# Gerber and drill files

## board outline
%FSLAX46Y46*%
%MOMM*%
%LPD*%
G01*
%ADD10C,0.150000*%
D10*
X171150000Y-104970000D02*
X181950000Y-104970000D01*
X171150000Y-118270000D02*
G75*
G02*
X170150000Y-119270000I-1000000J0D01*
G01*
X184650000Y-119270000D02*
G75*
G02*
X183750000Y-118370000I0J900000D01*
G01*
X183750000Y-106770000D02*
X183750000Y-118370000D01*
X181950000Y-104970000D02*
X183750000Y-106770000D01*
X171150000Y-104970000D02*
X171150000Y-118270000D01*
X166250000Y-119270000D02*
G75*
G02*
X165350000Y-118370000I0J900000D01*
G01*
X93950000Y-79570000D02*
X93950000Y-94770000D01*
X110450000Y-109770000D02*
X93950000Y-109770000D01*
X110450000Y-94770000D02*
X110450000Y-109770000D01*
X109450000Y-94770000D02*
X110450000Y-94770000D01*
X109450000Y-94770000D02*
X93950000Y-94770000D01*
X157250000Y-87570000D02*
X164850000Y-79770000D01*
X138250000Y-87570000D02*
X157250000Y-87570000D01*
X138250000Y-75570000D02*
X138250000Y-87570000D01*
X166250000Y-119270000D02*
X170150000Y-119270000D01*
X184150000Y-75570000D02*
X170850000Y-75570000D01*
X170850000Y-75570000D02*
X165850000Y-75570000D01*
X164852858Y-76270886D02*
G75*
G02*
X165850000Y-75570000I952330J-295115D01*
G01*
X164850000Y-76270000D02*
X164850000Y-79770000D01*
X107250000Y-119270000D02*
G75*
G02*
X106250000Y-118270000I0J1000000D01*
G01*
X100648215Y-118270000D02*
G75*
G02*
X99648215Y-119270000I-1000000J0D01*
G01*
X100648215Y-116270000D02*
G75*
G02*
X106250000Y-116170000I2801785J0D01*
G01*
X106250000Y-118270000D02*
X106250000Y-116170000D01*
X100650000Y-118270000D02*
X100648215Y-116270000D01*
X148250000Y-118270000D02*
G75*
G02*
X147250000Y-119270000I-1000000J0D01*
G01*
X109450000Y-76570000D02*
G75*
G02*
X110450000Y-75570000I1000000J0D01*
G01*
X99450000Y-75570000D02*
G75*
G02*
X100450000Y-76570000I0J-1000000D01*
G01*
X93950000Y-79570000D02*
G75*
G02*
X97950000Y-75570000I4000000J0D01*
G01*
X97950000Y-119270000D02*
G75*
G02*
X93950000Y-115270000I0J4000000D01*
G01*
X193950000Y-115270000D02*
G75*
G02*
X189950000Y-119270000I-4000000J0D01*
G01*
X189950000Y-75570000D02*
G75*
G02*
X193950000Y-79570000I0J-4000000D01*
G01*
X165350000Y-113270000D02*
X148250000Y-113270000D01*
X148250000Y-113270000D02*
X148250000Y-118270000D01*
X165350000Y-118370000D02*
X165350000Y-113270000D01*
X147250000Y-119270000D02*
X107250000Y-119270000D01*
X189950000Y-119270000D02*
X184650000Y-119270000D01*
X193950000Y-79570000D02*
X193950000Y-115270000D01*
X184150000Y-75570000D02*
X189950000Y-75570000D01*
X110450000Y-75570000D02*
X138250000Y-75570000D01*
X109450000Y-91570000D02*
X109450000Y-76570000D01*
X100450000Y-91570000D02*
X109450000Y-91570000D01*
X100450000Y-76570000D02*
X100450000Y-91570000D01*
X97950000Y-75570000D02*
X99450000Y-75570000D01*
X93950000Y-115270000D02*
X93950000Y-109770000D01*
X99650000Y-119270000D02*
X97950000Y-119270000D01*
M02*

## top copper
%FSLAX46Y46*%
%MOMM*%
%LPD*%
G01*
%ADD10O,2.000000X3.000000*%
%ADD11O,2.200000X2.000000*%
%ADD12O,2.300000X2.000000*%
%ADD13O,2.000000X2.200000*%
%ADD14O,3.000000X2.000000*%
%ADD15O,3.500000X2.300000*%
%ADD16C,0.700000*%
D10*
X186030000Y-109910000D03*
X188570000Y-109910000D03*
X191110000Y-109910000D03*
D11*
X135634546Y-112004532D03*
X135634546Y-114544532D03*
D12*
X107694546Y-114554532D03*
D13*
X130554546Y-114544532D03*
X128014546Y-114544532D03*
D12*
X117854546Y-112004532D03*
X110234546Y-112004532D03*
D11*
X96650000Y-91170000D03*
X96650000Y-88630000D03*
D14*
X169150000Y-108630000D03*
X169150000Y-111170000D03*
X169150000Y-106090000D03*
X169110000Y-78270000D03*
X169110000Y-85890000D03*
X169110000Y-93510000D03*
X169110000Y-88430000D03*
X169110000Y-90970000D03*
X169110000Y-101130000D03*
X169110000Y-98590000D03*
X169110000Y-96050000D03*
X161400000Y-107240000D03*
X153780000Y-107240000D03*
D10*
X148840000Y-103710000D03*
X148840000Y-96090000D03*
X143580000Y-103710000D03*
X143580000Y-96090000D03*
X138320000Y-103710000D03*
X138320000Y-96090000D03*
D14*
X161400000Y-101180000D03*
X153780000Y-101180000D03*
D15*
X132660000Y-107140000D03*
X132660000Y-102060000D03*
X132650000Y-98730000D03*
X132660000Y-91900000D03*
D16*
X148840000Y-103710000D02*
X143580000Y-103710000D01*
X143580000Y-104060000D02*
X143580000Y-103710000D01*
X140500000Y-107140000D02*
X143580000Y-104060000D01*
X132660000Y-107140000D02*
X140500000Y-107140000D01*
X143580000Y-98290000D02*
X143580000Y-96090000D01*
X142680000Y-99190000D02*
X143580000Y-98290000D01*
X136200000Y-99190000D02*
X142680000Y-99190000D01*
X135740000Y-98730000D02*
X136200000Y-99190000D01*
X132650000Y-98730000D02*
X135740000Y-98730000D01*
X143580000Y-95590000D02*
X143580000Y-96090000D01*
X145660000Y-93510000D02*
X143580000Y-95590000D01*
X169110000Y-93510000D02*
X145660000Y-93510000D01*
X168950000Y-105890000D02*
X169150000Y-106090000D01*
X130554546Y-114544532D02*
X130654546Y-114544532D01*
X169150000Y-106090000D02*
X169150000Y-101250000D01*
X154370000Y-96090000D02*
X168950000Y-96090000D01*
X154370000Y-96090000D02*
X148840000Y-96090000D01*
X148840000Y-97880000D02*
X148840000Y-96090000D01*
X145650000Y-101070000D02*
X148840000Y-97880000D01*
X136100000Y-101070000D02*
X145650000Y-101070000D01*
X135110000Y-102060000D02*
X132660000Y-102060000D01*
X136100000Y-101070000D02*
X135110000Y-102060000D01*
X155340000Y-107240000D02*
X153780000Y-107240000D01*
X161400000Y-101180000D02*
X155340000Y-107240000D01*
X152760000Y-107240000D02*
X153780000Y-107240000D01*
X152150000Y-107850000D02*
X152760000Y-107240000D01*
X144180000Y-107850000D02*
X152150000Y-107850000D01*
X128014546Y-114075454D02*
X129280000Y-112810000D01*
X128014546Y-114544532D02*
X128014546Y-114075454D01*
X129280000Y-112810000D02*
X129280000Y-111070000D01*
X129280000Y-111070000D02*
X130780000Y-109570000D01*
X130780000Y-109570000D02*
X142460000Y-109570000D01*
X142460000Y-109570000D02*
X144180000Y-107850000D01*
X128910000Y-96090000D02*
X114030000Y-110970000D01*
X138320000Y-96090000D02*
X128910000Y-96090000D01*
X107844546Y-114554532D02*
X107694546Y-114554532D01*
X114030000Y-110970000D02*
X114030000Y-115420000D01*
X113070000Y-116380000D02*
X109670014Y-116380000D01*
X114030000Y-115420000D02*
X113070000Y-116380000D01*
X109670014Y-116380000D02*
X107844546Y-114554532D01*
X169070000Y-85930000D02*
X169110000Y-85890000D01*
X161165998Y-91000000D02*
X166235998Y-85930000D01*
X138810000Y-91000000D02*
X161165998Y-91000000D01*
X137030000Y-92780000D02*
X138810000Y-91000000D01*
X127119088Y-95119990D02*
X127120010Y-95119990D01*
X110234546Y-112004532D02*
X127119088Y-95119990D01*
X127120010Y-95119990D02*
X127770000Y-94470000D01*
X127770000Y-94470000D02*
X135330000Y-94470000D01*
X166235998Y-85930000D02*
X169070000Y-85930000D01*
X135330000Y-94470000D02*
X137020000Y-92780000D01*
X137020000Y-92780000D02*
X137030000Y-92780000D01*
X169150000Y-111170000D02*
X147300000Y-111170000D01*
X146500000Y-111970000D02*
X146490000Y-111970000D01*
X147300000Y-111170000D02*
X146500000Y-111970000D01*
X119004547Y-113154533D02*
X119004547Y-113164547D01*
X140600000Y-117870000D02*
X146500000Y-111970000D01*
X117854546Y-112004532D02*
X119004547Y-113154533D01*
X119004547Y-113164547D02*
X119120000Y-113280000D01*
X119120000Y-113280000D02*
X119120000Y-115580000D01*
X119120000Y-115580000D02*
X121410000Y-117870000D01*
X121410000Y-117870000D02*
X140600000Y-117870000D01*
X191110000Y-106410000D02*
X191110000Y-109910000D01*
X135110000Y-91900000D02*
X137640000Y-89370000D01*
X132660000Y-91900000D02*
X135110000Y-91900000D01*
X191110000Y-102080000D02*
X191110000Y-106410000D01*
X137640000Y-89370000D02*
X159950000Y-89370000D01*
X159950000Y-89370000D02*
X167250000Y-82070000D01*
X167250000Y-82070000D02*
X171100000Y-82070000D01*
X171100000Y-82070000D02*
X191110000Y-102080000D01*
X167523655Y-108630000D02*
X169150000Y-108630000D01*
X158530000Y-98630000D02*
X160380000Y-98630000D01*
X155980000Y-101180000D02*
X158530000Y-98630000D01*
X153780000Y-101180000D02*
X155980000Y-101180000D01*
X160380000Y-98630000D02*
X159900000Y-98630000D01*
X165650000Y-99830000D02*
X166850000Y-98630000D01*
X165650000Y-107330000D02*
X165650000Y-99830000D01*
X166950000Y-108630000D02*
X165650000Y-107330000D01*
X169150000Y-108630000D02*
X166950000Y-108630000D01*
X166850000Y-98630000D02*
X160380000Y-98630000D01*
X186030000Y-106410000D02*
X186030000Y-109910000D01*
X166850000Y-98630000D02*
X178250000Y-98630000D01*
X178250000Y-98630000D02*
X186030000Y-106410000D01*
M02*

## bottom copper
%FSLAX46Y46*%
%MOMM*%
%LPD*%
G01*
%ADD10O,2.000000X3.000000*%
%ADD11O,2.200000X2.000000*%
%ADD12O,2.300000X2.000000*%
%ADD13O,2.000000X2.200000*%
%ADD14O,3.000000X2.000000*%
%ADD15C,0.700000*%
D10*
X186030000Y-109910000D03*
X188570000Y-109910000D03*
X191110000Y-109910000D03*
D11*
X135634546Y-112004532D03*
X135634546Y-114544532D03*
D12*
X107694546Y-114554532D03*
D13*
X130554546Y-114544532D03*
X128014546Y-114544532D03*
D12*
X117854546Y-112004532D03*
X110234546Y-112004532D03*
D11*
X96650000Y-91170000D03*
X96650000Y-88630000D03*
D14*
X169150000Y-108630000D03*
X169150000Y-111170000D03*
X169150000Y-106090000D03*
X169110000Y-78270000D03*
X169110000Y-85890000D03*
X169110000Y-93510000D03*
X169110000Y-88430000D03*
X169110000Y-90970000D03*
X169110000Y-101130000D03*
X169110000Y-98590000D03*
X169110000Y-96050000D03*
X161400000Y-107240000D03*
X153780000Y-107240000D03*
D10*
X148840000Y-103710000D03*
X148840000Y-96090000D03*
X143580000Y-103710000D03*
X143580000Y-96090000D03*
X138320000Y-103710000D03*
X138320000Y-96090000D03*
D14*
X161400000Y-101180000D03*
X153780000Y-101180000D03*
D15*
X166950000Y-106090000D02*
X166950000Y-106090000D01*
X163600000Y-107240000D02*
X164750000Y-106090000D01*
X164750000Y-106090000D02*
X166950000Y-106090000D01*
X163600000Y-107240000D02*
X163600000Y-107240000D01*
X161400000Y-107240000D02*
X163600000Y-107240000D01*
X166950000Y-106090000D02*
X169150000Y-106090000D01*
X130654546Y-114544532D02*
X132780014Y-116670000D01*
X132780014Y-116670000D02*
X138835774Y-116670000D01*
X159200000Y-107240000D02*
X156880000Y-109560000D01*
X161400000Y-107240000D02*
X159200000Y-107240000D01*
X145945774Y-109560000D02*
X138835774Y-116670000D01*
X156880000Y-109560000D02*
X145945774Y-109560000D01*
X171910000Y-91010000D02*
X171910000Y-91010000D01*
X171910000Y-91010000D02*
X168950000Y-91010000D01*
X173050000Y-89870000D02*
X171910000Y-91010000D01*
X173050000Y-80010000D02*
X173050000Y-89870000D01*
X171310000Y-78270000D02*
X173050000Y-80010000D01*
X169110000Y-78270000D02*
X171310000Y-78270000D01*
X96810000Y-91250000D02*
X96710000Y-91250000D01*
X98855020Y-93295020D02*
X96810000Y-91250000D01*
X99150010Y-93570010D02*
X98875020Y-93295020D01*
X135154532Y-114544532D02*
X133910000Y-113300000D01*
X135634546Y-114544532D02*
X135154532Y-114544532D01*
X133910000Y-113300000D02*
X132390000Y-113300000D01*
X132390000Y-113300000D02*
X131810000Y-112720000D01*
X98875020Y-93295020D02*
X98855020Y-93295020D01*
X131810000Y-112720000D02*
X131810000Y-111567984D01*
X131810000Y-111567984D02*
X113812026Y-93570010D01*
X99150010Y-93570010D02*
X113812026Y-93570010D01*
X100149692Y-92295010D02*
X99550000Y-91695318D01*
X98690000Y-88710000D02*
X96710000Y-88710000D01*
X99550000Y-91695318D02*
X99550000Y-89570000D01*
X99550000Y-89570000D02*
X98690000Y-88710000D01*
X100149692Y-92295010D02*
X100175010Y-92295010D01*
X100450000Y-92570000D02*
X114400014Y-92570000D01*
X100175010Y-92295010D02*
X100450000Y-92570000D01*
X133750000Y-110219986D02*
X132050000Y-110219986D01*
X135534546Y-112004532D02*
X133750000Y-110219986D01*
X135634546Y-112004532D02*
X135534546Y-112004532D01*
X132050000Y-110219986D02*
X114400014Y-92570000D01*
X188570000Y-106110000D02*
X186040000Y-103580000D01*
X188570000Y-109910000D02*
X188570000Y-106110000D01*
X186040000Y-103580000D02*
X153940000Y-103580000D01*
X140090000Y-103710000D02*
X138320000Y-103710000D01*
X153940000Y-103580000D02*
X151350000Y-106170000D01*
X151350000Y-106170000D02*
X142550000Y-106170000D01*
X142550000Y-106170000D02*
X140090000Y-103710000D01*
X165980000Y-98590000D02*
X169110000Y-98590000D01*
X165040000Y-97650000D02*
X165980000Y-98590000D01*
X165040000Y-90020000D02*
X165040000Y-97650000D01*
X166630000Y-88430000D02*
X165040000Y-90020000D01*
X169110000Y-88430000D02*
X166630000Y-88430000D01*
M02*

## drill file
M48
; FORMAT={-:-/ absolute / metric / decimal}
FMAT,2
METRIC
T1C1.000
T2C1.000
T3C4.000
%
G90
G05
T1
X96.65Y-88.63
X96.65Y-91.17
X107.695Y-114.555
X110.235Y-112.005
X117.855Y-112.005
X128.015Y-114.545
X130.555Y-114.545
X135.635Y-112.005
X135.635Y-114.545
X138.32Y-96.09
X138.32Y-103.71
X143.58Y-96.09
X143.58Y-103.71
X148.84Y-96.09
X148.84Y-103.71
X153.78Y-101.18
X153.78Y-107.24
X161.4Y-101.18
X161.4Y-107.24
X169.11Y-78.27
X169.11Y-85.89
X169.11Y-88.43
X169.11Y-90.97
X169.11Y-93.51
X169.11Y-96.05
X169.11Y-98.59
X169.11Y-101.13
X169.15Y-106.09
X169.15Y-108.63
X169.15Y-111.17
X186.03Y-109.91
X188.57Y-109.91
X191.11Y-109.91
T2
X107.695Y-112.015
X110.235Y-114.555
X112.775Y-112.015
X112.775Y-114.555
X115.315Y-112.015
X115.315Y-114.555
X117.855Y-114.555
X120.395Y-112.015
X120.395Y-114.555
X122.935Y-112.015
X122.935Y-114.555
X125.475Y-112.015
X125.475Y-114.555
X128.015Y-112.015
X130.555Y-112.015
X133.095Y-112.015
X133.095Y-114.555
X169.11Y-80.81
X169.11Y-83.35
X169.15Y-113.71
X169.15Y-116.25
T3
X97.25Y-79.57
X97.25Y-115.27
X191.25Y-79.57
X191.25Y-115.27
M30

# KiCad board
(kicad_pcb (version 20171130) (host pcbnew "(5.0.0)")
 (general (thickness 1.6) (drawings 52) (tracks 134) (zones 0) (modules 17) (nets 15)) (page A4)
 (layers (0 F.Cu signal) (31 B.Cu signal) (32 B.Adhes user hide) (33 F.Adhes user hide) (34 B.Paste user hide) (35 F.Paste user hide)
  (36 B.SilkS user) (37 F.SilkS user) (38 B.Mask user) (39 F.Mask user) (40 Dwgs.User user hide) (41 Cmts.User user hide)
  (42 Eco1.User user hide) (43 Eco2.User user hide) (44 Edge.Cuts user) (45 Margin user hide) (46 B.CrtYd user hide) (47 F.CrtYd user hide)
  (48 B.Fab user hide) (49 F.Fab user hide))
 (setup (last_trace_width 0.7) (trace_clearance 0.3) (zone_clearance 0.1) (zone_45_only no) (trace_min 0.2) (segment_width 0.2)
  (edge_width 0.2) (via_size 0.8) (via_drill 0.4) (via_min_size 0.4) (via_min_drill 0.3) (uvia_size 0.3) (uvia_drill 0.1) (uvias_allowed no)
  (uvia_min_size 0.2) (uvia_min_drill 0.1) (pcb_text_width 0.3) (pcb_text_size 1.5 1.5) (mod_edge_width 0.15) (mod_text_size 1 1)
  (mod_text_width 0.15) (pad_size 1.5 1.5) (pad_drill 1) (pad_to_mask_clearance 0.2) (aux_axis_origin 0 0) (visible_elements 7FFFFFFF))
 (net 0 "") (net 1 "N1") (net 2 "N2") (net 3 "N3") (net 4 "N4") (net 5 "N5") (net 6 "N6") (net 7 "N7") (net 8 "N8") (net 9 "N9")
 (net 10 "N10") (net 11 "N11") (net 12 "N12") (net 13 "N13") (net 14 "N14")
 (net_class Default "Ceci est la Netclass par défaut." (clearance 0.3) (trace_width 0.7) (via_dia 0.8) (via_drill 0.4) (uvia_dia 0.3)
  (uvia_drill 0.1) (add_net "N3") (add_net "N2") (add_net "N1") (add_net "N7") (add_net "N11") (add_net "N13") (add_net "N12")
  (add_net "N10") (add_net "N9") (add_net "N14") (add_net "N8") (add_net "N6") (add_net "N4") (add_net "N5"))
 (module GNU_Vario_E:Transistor (layer F.Cu) (at 193.65 107.37 180)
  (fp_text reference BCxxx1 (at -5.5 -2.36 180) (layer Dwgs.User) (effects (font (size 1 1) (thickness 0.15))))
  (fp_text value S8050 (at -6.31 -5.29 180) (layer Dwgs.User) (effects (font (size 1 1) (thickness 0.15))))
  (pad 3 thru_hole oval (at 7.62 -2.54 180) (size 2 3) (drill 1) (layers *.Cu *.Mask) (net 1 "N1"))
  (pad 2 thru_hole oval (at 5.08 -2.54 180) (size 2 3) (drill 1) (layers *.Cu *.Mask) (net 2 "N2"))
  (pad 1 thru_hole oval (at 2.54 -2.54 180) (size 2 3) (drill 1) (layers *.Cu *.Mask) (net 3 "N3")))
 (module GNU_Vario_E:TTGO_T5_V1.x (layer F.Cu) (at 136.184546 112.224532 90)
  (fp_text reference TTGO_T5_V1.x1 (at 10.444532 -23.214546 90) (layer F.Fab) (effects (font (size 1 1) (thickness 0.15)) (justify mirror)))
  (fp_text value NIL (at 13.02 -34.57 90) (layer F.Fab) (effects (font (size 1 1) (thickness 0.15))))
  (pad "" np_thru_hole circle (at 0.21 -28.49 90) (size 1 1) (drill 1) (layers *.Cu *.Mask))
  (pad "" np_thru_hole circle (at 0.21 -23.41 90) (size 1 1) (drill 1) (layers *.Cu *.Mask))
  (pad "" np_thru_hole circle (at 0.21 -20.87 90) (size 1 1) (drill 1) (layers *.Cu *.Mask))
  (pad "" np_thru_hole circle (at -2.33 -3.09 90) (size 1 1) (drill 1) (layers *.Cu *.Mask))
  (pad "" np_thru_hole circle (at 0.21 -3.09 90) (size 1 1) (drill 1) (layers *.Cu *.Mask))
  (pad "" np_thru_hole circle (at 0.21 -5.63 90) (size 1 1) (drill 1) (layers *.Cu *.Mask))
  (pad "" np_thru_hole circle (at 0.21 -15.79 90) (size 1 1) (drill 1) (layers *.Cu *.Mask))
  (pad "" np_thru_hole circle (at 0.21 -13.25 90) (size 1 1) (drill 1) (layers *.Cu *.Mask))
  (pad "" np_thru_hole circle (at 0.21 -8.17 90) (size 1 1) (drill 1) (layers *.Cu *.Mask))
  (pad "" np_thru_hole circle (at 0.21 -10.71 90) (size 1 1) (drill 1) (layers *.Cu *.Mask))
  (pad "" np_thru_hole circle (at -2.33 -10.71 90) (size 1 1) (drill 1) (layers *.Cu *.Mask))
  (pad "" np_thru_hole circle (at -2.33 -13.25 90) (size 1 1) (drill 1) (layers *.Cu *.Mask))
  (pad "" np_thru_hole circle (at -2.33 -15.79 90) (size 1 1) (drill 1) (layers *.Cu *.Mask))
  (pad "" np_thru_hole circle (at -2.33 -18.33 90) (size 1 1) (drill 1) (layers *.Cu *.Mask))
  (pad "" np_thru_hole circle (at -2.33 -20.87 90) (size 1 1) (drill 1) (layers *.Cu *.Mask))
  (pad "" np_thru_hole circle (at -2.33 -23.41 90) (size 1 1) (drill 1) (layers *.Cu *.Mask))
  (pad "" np_thru_hole circle (at -2.33 -25.95 90) (size 1 1) (drill 1) (layers *.Cu *.Mask))
  (pad 13 thru_hole oval (at 0.22 -0.55 90) (size 2 2.2) (drill 1) (layers *.Cu *.Mask) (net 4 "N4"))
  (pad 1 thru_hole oval (at -2.32 -0.55 90) (size 2 2.2) (drill 1) (layers *.Cu *.Mask) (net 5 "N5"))
  (pad 12 thru_hole oval (at -2.33 -28.49 90) (size 2 2.3) (drill 1) (layers *.Cu *.Mask) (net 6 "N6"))
  (pad 3 thru_hole oval (at -2.32 -5.63 90) (size 2.2 2) (drill 1) (layers *.Cu *.Mask) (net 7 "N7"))
  (pad 4 thru_hole oval (at -2.32 -8.17 90) (size 2.2 2) (drill 1) (layers *.Cu *.Mask) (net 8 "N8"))
  (pad 20 thru_hole oval (at 0.22 -18.33 90) (size 2 2.3) (drill 1) (layers *.Cu *.Mask) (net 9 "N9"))
  (pad 23 thru_hole oval (at 0.22 -25.95 90) (size 2 2.3) (drill 1) (layers *.Cu *.Mask) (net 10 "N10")))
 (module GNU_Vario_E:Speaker (layer F.Cu) (at 99.19 93.71 90)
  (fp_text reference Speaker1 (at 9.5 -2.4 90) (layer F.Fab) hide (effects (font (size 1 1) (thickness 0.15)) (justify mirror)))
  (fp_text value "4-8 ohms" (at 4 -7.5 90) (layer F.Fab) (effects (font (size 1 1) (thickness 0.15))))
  (pad 2 thru_hole oval (at 2.54 -2.54 90) (size 2 2.2) (drill 1) (layers *.Cu *.Mask) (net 5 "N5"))
  (pad 1 thru_hole oval (at 5.08 -2.54 90) (size 2 2.2) (drill 1) (layers *.Cu *.Mask) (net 4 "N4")))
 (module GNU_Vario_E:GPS (layer F.Cu) (at 169.15 106.09 270)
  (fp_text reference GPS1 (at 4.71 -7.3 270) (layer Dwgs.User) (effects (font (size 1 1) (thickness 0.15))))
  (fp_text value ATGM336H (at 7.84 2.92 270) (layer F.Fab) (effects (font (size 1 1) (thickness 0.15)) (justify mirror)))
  (pad 2 thru_hole oval (at 2.54 0 270) (size 2 3) (drill 1) (layers *.Cu *.Mask) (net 1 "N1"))
  (pad 3 thru_hole oval (at 5.08 0 270) (size 2 3) (drill 1) (layers *.Cu *.Mask) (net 9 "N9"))
  (pad 1 thru_hole oval (at 0 0 270) (size 2 3) (drill 1) (layers *.Cu *.Mask) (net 7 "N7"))
  (pad "" np_thru_hole circle (at 7.62 0 270) (size 1 1) (drill 1) (layers *.Cu *.Mask))
  (pad "" np_thru_hole circle (at 10.16 0 270) (size 1 1) (drill 1) (layers *.Cu *.Mask)))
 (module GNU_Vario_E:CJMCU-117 (layer F.Cu) (at 171.65 90.97 90)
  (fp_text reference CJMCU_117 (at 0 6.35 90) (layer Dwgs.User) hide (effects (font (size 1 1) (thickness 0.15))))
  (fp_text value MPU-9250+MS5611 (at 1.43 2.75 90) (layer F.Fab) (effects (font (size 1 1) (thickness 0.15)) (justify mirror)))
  (pad 10 thru_hole oval (at 12.7 -2.54 90) (size 2 3) (drill 1) (layers *.Cu *.Mask) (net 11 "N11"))
  (pad 7 thru_hole oval (at 5.08 -2.54 90) (size 2 3) (drill 1) (layers *.Cu *.Mask) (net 10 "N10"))
  (pad 4 thru_hole oval (at -2.54 -2.54 90) (size 2 3) (drill 1) (layers *.Cu *.Mask) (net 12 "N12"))
  (pad 6 thru_hole oval (at 2.54 -2.54 90) (size 2 3) (drill 1) (layers *.Cu *.Mask) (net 1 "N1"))
  (pad 5 thru_hole oval (at 0 -2.54 90) (size 2 3) (drill 1) (layers *.Cu *.Mask) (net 11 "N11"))
  (pad 1 thru_hole oval (at -10.16 -2.54 90) (size 2 3) (drill 1) (layers *.Cu *.Mask) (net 7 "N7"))
  (pad 2 thru_hole oval (at -7.62 -2.54 90) (size 2 3) (drill 1) (layers *.Cu *.Mask) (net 1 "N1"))
  (pad 3 thru_hole oval (at -5.08 -2.54 90) (size 2 3) (drill 1) (layers *.Cu *.Mask) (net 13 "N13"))
  (pad "" np_thru_hole circle (at 7.62 -2.54 90) (size 1 1) (drill 1) (layers *.Cu *.Mask))
  (pad "" np_thru_hole circle (at 10.16 -2.54 90) (size 1 1) (drill 1) (layers *.Cu *.Mask)))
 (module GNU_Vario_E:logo (layer F.Cu) (at 115.96 84.56 90)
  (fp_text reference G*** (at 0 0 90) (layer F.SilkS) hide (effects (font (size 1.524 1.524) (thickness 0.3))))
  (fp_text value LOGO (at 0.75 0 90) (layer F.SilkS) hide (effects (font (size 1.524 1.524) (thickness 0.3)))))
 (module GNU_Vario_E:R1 (layer F.Cu) (at 153.78 107.24 270)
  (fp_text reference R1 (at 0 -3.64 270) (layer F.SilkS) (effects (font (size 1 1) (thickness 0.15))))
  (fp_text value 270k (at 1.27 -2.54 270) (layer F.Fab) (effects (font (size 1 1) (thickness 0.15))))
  (pad 2 thru_hole oval (at 0 -7.62 270) (size 2 3) (drill 1) (layers *.Cu *.Mask) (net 7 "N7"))
  (pad 1 thru_hole oval (at 0 0 270) (size 2 3) (drill 1) (layers *.Cu *.Mask) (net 8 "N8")))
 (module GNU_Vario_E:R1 (layer F.Cu) (at 148.84 96.09 180)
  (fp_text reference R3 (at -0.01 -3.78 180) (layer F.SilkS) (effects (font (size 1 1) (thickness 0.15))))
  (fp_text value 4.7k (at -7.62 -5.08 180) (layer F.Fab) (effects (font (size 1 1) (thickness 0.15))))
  (pad 2 thru_hole oval (at 0 -7.62 180) (size 2 3) (drill 1) (layers *.Cu *.Mask) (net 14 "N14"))
  (pad 1 thru_hole oval (at 0 0 180) (size 2 3) (drill 1) (layers *.Cu *.Mask) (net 13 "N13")))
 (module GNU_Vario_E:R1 (layer F.Cu) (at 143.58 96.09 180)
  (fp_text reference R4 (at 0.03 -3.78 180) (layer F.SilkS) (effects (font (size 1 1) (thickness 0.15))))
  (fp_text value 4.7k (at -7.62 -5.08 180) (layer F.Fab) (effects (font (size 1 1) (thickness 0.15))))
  (pad 2 thru_hole oval (at 0 -7.62 180) (size 2 3) (drill 1) (layers *.Cu *.Mask) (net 14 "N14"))
  (pad 1 thru_hole oval (at 0 0 180) (size 2 3) (drill 1) (layers *.Cu *.Mask) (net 12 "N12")))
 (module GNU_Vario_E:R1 (layer F.Cu) (at 138.32 96.09 180)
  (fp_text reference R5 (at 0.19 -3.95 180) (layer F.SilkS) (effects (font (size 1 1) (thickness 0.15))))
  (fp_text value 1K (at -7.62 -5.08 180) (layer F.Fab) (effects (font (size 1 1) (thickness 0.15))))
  (pad 2 thru_hole oval (at 0 -7.62 180) (size 2 3) (drill 1) (layers *.Cu *.Mask) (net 2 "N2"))
  (pad 1 thru_hole oval (at 0 0 180) (size 2 3) (drill 1) (layers *.Cu *.Mask) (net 6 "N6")))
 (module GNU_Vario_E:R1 (layer F.Cu) (at 153.78 101.18 270)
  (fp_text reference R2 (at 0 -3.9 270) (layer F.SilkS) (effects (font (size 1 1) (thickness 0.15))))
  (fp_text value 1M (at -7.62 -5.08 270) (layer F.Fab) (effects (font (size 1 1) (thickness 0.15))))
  (pad 2 thru_hole oval (at 0 -7.62 270) (size 2 3) (drill 1) (layers *.Cu *.Mask) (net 8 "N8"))
  (pad 1 thru_hole oval (at 0 0 270) (size 2 3) (drill 1) (layers *.Cu *.Mask) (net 1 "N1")))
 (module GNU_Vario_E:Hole (layer F.Cu) (at 97.25 115.27)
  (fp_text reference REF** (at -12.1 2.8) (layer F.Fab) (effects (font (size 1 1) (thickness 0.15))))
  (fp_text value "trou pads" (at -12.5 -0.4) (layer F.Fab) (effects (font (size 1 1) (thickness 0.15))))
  (pad "" np_thru_hole circle (at 0 0) (size 4 4) (drill 4) (layers *.Cu *.Mask)))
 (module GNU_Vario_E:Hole (layer F.Cu) (at 97.25 79.57)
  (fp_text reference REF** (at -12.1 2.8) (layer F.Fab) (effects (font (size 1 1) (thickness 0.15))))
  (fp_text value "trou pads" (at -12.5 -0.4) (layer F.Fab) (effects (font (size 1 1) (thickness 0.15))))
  (pad "" np_thru_hole circle (at 0 0) (size 4 4) (drill 4) (layers *.Cu *.Mask)))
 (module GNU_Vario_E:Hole (layer F.Cu) (at 191.25 79.57)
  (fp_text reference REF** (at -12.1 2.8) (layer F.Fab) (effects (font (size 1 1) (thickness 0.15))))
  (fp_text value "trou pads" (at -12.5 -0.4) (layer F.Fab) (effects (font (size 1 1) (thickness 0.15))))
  (pad "" np_thru_hole circle (at 0 0) (size 4 4) (drill 4) (layers *.Cu *.Mask)))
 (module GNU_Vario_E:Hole (layer F.Cu) (at 191.25 115.27)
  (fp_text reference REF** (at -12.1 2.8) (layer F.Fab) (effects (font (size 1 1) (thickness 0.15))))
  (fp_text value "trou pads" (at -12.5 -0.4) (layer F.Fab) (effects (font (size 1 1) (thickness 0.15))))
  (pad "" np_thru_hole circle (at 0 0) (size 4 4) (drill 4) (layers *.Cu *.Mask)))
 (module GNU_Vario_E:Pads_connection (layer F.Cu) (at 132.66 94.44)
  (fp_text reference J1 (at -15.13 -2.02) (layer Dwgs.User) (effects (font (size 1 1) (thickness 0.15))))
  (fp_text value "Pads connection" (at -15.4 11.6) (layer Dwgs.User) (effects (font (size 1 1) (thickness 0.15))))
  (pad 5 smd oval (at 0 12.7) (size 3.5 2.3) (layers F.Cu F.Mask) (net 14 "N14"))
  (pad 4 smd oval (at 0 7.62) (size 3.5 2.3) (layers F.Cu F.Mask) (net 13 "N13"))
  (pad 3 smd oval (at -0.01 4.29) (size 3.5 2.3) (layers F.Cu F.Mask) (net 12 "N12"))
  (pad 1 smd oval (at 0 -2.54) (size 3.5 2.3) (layers F.Cu F.Mask) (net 3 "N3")))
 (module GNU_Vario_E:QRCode (layer B.Cu) (at 125.16 85.57)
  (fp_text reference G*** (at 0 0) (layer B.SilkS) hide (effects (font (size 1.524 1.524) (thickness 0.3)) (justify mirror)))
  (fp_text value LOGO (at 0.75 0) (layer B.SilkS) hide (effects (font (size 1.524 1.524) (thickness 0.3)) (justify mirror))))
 (gr_line (start 171.15 104.97) (end 181.95 104.97) (layer Edge.Cuts) (width 0.15))
 (gr_arc (start 170.15 118.27) (end 170.15 119.27) (angle -90) (layer Edge.Cuts) (width 0.15))
 (gr_arc (start 184.65 118.37) (end 183.75 118.37) (angle -90) (layer Edge.Cuts) (width 0.15))
 (gr_line (start 183.75 106.77) (end 183.75 118.37) (layer Edge.Cuts) (width 0.15))
 (gr_line (start 181.95 104.97) (end 183.75 106.77) (layer Edge.Cuts) (width 0.15))
 (gr_line (start 171.15 104.97) (end 171.15 118.27) (layer Edge.Cuts) (width 0.15))
 (gr_arc (start 166.25 118.37) (end 165.35 118.37) (angle -90) (layer Edge.Cuts) (width 0.15))
 (gr_line (start 93.95 79.57) (end 93.95 94.77) (layer Edge.Cuts) (width 0.15))
 (gr_line (start 110.45 109.77) (end 93.95 109.77) (layer Edge.Cuts) (width 0.15))
 (gr_line (start 110.45 94.77) (end 110.45 109.77) (layer Edge.Cuts) (width 0.15))
 (gr_line (start 109.45 94.77) (end 110.45 94.77) (layer Edge.Cuts) (width 0.15))
 (gr_line (start 109.45 94.77) (end 93.95 94.77) (layer Edge.Cuts) (width 0.15))
 (gr_line (start 157.25 87.57) (end 164.85 79.77) (layer Edge.Cuts) (width 0.15))
 (gr_line (start 138.25 87.57) (end 157.25 87.57) (layer Edge.Cuts) (width 0.15))
 (gr_line (start 138.25 75.57) (end 138.25 87.57) (layer Edge.Cuts) (width 0.15))
 (gr_line (start 166.25 119.27) (end 170.15 119.27) (layer Edge.Cuts) (width 0.15))
 (gr_line (start 184.15 75.57) (end 170.85 75.57) (layer Edge.Cuts) (width 0.15))
 (gr_line (start 170.85 75.57) (end 165.85 75.57) (layer Edge.Cuts) (width 0.15))
 (gr_arc (start 165.805188 76.566001) (end 165.85 75.57) (angle -75.35856355) (layer Edge.Cuts) (width 0.15))
 (gr_line (start 164.85 76.27) (end 164.85 79.77) (layer Edge.Cuts) (width 0.15))
 (gr_arc (start 107.25 118.27) (end 106.25 118.27) (angle -90) (layer Edge.Cuts) (width 0.15))
 (gr_arc (start 99.648215 118.27) (end 99.648215 119.27) (angle -90) (layer Edge.Cuts) (width 0.15))
 (gr_arc (start 103.45 116.27) (end 106.25 116.17) (angle -177.9545915) (layer Edge.Cuts) (width 0.15))
 (gr_line (start 106.25 118.27) (end 106.25 116.17) (layer Edge.Cuts) (width 0.15))
 (gr_line (start 100.65 118.27) (end 100.648215 116.27) (layer Edge.Cuts) (width 0.15))
 (gr_arc (start 147.25 118.27) (end 147.25 119.27) (angle -90) (layer Edge.Cuts) (width 0.15))
 (gr_arc (start 110.45 76.57) (end 110.45 75.57) (angle -90) (layer Edge.Cuts) (width 0.15))
 (gr_arc (start 99.45 76.57) (end 100.45 76.57) (angle -90) (layer Edge.Cuts) (width 0.15))
 (gr_arc (start 97.95 79.57) (end 97.95 75.57) (angle -90) (layer Edge.Cuts) (width 0.15))
 (gr_arc (start 97.95 115.27) (end 93.95 115.27) (angle -90) (layer Edge.Cuts) (width 0.15))
 (gr_arc (start 189.95 115.27) (end 189.95 119.27) (angle -90) (layer Edge.Cuts) (width 0.15))
 (gr_arc (start 189.95 79.57) (end 193.95 79.57) (angle -90) (layer Edge.Cuts) (width 0.15))
 (gr_line (start 165.35 113.27) (end 148.25 113.27) (layer Edge.Cuts) (width 0.15))
 (gr_line (start 148.25 113.27) (end 148.25 118.27) (layer Edge.Cuts) (width 0.15))
 (gr_line (start 165.35 118.37) (end 165.35 113.27) (layer Edge.Cuts) (width 0.15))
 (gr_line (start 147.25 119.27) (end 107.25 119.27) (layer Edge.Cuts) (width 0.15))
 (gr_line (start 189.95 119.27) (end 184.65 119.27) (layer Edge.Cuts) (width 0.15))
 (gr_line (start 193.95 79.57) (end 193.95 115.27) (layer Edge.Cuts) (width 0.15))
 (gr_line (start 184.15 75.57) (end 189.95 75.57) (layer Edge.Cuts) (width 0.15))
 (gr_line (start 110.45 75.57) (end 138.25 75.57) (layer Edge.Cuts) (width 0.15))
 (gr_line (start 109.45 91.57) (end 109.45 76.57) (layer Edge.Cuts) (width 0.15))
 (gr_line (start 100.45 91.57) (end 109.45 91.57) (layer Edge.Cuts) (width 0.15))
 (gr_line (start 100.45 76.57) (end 100.45 91.57) (layer Edge.Cuts) (width 0.15))
 (gr_line (start 97.95 75.57) (end 99.45 75.57) (layer Edge.Cuts) (width 0.15))
 (gr_line (start 93.95 115.27) (end 93.95 109.77) (layer Edge.Cuts) (width 0.15))
 (gr_line (start 99.65 119.27) (end 97.95 119.27) (layer Edge.Cuts) (width 0.15))
 (segment (start 148.84 103.71) (end 143.58 103.71) (width 0.7) (layer F.Cu) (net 14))
 (segment (start 143.58 104.06) (end 143.58 103.71) (width 0.7) (layer F.Cu) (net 14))
 (segment (start 140.5 107.14) (end 143.58 104.06) (width 0.7) (layer F.Cu) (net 14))
 (segment (start 132.66 107.14) (end 140.5 107.14) (width 0.7) (layer F.Cu) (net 14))
 (segment (start 143.58 98.29) (end 143.58 96.09) (width 0.7) (layer F.Cu) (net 12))
 (segment (start 142.68 99.19) (end 143.58 98.29) (width 0.7) (layer F.Cu) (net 12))
 (segment (start 136.2 99.19) (end 142.68 99.19) (width 0.7) (layer F.Cu) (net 12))
 (segment (start 135.74 98.73) (end 136.2 99.19) (width 0.7) (layer F.Cu) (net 12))
 (segment (start 132.65 98.73) (end 135.74 98.73) (width 0.7) (layer F.Cu) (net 12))
 (segment (start 143.58 95.59) (end 143.58 96.09) (width 0.7) (layer F.Cu) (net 12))
 (segment (start 145.66 93.51) (end 143.58 95.59) (width 0.7) (layer F.Cu) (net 12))
 (segment (start 169.11 93.51) (end 145.66 93.51) (width 0.7) (layer F.Cu) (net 12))
 (segment (start 168.95 105.89) (end 169.15 106.09) (width 0.7) (layer F.Cu) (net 7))
 (segment (start 166.95 106.09) (end 166.95 106.09) (width 0.7) (layer B.Cu) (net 7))
 (segment (start 163.6 107.24) (end 164.75 106.09) (width 0.7) (layer B.Cu) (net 7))
 (segment (start 164.75 106.09) (end 166.95 106.09) (width 0.7) (layer B.Cu) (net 7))
 (segment (start 163.6 107.24) (end 163.6 107.24) (width 0.7) (layer B.Cu) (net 7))
 (segment (start 161.4 107.24) (end 163.6 107.24) (width 0.7) (layer B.Cu) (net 7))
 (segment (start 166.95 106.09) (end 169.15 106.09) (width 0.7) (layer B.Cu) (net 7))
 (segment (start 130.654546 114.544532) (end 132.780014 116.67) (width 0.7) (layer B.Cu) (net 7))
 (segment (start 130.554546 114.544532) (end 130.654546 114.544532) (width 0.7) (layer F.Cu) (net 7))
 (segment (start 132.780014 116.67) (end 138.835774 116.67) (width 0.7) (layer B.Cu) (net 7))
 (segment (start 169.15 106.09) (end 169.15 101.25) (width 0.7) (layer F.Cu) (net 7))
 (segment (start 159.2 107.24) (end 156.88 109.56) (width 0.7) (layer B.Cu) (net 7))
 (segment (start 161.4 107.24) (end 159.2 107.24) (width 0.7) (layer B.Cu) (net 7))
 (segment (start 145.945774 109.56) (end 138.835774 116.67) (width 0.7) (layer B.Cu) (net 7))
 (segment (start 156.88 109.56) (end 145.945774 109.56) (width 0.7) (layer B.Cu) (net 7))
 (segment (start 154.37 96.09) (end 168.95 96.09) (width 0.7) (layer F.Cu) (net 13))
 (segment (start 154.37 96.09) (end 148.84 96.09) (width 0.7) (layer F.Cu) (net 13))
 (segment (start 148.84 97.88) (end 148.84 96.09) (width 0.7) (layer F.Cu) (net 13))
 (segment (start 145.65 101.07) (end 148.84 97.88) (width 0.7) (layer F.Cu) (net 13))
 (segment (start 136.1 101.07) (end 145.65 101.07) (width 0.7) (layer F.Cu) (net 13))
 (segment (start 135.11 102.06) (end 132.66 102.06) (width 0.7) (layer F.Cu) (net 13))
 (segment (start 136.1 101.07) (end 135.11 102.06) (width 0.7) (layer F.Cu) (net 13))
 (segment (start 155.34 107.24) (end 153.78 107.24) (width 0.7) (layer F.Cu) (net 8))
 (segment (start 161.4 101.18) (end 155.34 107.24) (width 0.7) (layer F.Cu) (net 8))
 (segment (start 152.76 107.24) (end 153.78 107.24) (width 0.7) (layer F.Cu) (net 8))
 (segment (start 152.15 107.85) (end 152.76 107.24) (width 0.7) (layer F.Cu) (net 8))
 (segment (start 144.18 107.85) (end 152.15 107.85) (width 0.7) (layer F.Cu) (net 8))
 (segment (start 128.014546 114.075454) (end 129.28 112.81) (width 0.7) (layer F.Cu) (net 8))
 (segment (start 128.014546 114.544532) (end 128.014546 114.075454) (width 0.7) (layer F.Cu) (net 8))
 (segment (start 129.28 112.81) (end 129.28 111.07) (width 0.7) (layer F.Cu) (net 8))
 (segment (start 129.28 111.07) (end 130.78 109.57) (width 0.7) (layer F.Cu) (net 8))
 (segment (start 130.78 109.57) (end 142.46 109.57) (width 0.7) (layer F.Cu) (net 8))
 (segment (start 142.46 109.57) (end 144.18 107.85) (width 0.7) (layer F.Cu) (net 8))
 (segment (start 128.91 96.09) (end 114.03 110.97) (width 0.7) (layer F.Cu) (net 6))
 (segment (start 138.32 96.09) (end 128.91 96.09) (width 0.7) (layer F.Cu) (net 6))
 (segment (start 107.844546 114.554532) (end 107.694546 114.554532) (width 0.7) (layer F.Cu) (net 6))
 (segment (start 114.03 110.97) (end 114.03 115.42) (width 0.7) (layer F.Cu) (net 6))
 (segment (start 113.07 116.38) (end 109.670014 116.38) (width 0.7) (layer F.Cu) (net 6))
 (segment (start 114.03 115.42) (end 113.07 116.38) (width 0.7) (layer F.Cu) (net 6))
 (segment (start 109.670014 116.38) (end 107.844546 114.554532) (width 0.7) (layer F.Cu) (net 6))
 (segment (start 171.91 91.01) (end 171.91 91.01) (width 0.7) (layer B.Cu) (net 11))
 (segment (start 171.91 91.01) (end 168.95 91.01) (width 0.7) (layer B.Cu) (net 11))
 (segment (start 173.05 89.87) (end 171.91 91.01) (width 0.7) (layer B.Cu) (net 11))
 (segment (start 173.05 80.01) (end 173.05 89.87) (width 0.7) (layer B.Cu) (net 11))
 (segment (start 171.31 78.27) (end 173.05 80.01) (width 0.7) (layer B.Cu) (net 11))
 (segment (start 169.11 78.27) (end 171.31 78.27) (width 0.7) (layer B.Cu) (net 11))
 (segment (start 169.07 85.93) (end 169.11 85.89) (width 0.7) (layer F.Cu) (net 10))
 (segment (start 161.165998 91) (end 166.235998 85.93) (width 0.7) (layer F.Cu) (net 10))
 (segment (start 138.81 91) (end 161.165998 91) (width 0.7) (layer F.Cu) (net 10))
 (segment (start 137.03 92.78) (end 138.81 91) (width 0.7) (layer F.Cu) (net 10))
 (segment (start 127.119088 95.11999) (end 127.12001 95.11999) (width 0.7) (layer F.Cu) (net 10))
 (segment (start 110.234546 112.004532) (end 127.119088 95.11999) (width 0.7) (layer F.Cu) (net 10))
 (segment (start 127.12001 95.11999) (end 127.77 94.47) (width 0.7) (layer F.Cu) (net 10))
 (segment (start 127.77 94.47) (end 135.33 94.47) (width 0.7) (layer F.Cu) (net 10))
 (segment (start 166.235998 85.93) (end 169.07 85.93) (width 0.7) (layer F.Cu) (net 10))
 (segment (start 135.33 94.47) (end 137.02 92.78) (width 0.7) (layer F.Cu) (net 10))
 (segment (start 137.02 92.78) (end 137.03 92.78) (width 0.7) (layer F.Cu) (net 10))
 (segment (start 169.15 111.17) (end 147.3 111.17) (width 0.7) (layer F.Cu) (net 9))
 (segment (start 146.5 111.97) (end 146.49 111.97) (width 0.7) (layer F.Cu) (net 9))
 (segment (start 147.3 111.17) (end 146.5 111.97) (width 0.7) (layer F.Cu) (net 9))
 (segment (start 119.004547 113.154533) (end 119.004547 113.164547) (width 0.7) (layer F.Cu) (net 9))
 (segment (start 140.6 117.87) (end 146.5 111.97) (width 0.7) (layer F.Cu) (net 9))
 (segment (start 117.854546 112.004532) (end 119.004547 113.154533) (width 0.7) (layer F.Cu) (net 9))
 (segment (start 119.004547 113.164547) (end 119.12 113.28) (width 0.7) (layer F.Cu) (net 9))
 (segment (start 119.12 113.28) (end 119.12 115.58) (width 0.7) (layer F.Cu) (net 9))
 (segment (start 119.12 115.58) (end 121.41 117.87) (width 0.7) (layer F.Cu) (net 9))
 (segment (start 121.41 117.87) (end 140.6 117.87) (width 0.7) (layer F.Cu) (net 9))
 (segment (start 96.81 91.25) (end 96.71 91.25) (width 0.7) (layer B.Cu) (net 5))
 (segment (start 98.85502 93.29502) (end 96.81 91.25) (width 0.7) (layer B.Cu) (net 5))
 (segment (start 99.15001 93.57001) (end 98.87502 93.29502) (width 0.7) (layer B.Cu) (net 5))
 (segment (start 135.154532 114.544532) (end 133.91 113.3) (width 0.7) (layer B.Cu) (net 5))
 (segment (start 135.634546 114.544532) (end 135.154532 114.544532) (width 0.7) (layer B.Cu) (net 5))
 (segment (start 133.91 113.3) (end 132.39 113.3) (width 0.7) (layer B.Cu) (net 5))
 (segment (start 132.39 113.3) (end 131.81 112.72) (width 0.7) (layer B.Cu) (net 5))
 (segment (start 98.87502 93.29502) (end 98.85502 93.29502) (width 0.7) (layer B.Cu) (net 5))
 (segment (start 131.81 112.72) (end 131.81 111.567984) (width 0.7) (layer B.Cu) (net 5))
 (segment (start 131.81 111.567984) (end 113.812026 93.57001) (width 0.7) (layer B.Cu) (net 5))
 (segment (start 99.15001 93.57001) (end 113.812026 93.57001) (width 0.7) (layer B.Cu) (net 5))
 (segment (start 100.149692 92.29501) (end 99.55 91.695318) (width 0.7) (layer B.Cu) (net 4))
 (segment (start 98.69 88.71) (end 96.71 88.71) (width 0.7) (layer B.Cu) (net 4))
 (segment (start 99.55 91.695318) (end 99.55 89.57) (width 0.7) (layer B.Cu) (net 4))
 (segment (start 99.55 89.57) (end 98.69 88.71) (width 0.7) (layer B.Cu) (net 4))
 (segment (start 100.149692 92.29501) (end 100.17501 92.29501) (width 0.7) (layer B.Cu) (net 4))
 (segment (start 100.45 92.57) (end 114.400014 92.57) (width 0.7) (layer B.Cu) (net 4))
 (segment (start 100.17501 92.29501) (end 100.45 92.57) (width 0.7) (layer B.Cu) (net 4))
 (segment (start 133.75 110.219986) (end 132.05 110.219986) (width 0.7) (layer B.Cu) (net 4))
 (segment (start 135.534546 112.004532) (end 133.75 110.219986) (width 0.7) (layer B.Cu) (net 4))
 (segment (start 135.634546 112.004532) (end 135.534546 112.004532) (width 0.7) (layer B.Cu) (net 4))
 (segment (start 132.05 110.219986) (end 114.400014 92.57) (width 0.7) (layer B.Cu) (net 4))
 (segment (start 191.11 106.41) (end 191.11 109.91) (width 0.7) (layer F.Cu) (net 3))
 (segment (start 135.11 91.9) (end 137.64 89.37) (width 0.7) (layer F.Cu) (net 3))
 (segment (start 132.66 91.9) (end 135.11 91.9) (width 0.7) (layer F.Cu) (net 3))
 (segment (start 191.11 102.08) (end 191.11 106.41) (width 0.7) (layer F.Cu) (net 3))
 (segment (start 137.64 89.37) (end 159.95 89.37) (width 0.7) (layer F.Cu) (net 3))
 (segment (start 159.95 89.37) (end 167.25 82.07) (width 0.7) (layer F.Cu) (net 3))
 (segment (start 167.25 82.07) (end 171.1 82.07) (width 0.7) (layer F.Cu) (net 3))
 (segment (start 171.1 82.07) (end 191.11 102.08) (width 0.7) (layer F.Cu) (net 3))
 (segment (start 188.57 106.11) (end 186.04 103.58) (width 0.7) (layer B.Cu) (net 2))
 (segment (start 188.57 109.91) (end 188.57 106.11) (width 0.7) (layer B.Cu) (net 2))
 (segment (start 186.04 103.58) (end 153.94 103.58) (width 0.7) (layer B.Cu) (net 2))
 (segment (start 140.09 103.71) (end 138.32 103.71) (width 0.7) (layer B.Cu) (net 2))
 (segment (start 153.94 103.58) (end 151.35 106.17) (width 0.7) (layer B.Cu) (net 2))
 (segment (start 151.35 106.17) (end 142.55 106.17) (width 0.7) (layer B.Cu) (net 2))
 (segment (start 142.55 106.17) (end 140.09 103.71) (width 0.7) (layer B.Cu) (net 2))
 (segment (start 167.523655 108.63) (end 169.15 108.63) (width 0.7) (layer F.Cu) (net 1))
 (segment (start 158.53 98.63) (end 160.38 98.63) (width 0.7) (layer F.Cu) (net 1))
 (segment (start 155.98 101.18) (end 158.53 98.63) (width 0.7) (layer F.Cu) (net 1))
 (segment (start 153.78 101.18) (end 155.98 101.18) (width 0.7) (layer F.Cu) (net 1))
 (segment (start 160.38 98.63) (end 159.9 98.63) (width 0.7) (layer F.Cu) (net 1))
 (segment (start 165.65 99.83) (end 166.85 98.63) (width 0.7) (layer F.Cu) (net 1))
 (segment (start 165.65 107.33) (end 165.65 99.83) (width 0.7) (layer F.Cu) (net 1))
 (segment (start 166.95 108.63) (end 165.65 107.33) (width 0.7) (layer F.Cu) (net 1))
 (segment (start 169.15 108.63) (end 166.95 108.63) (width 0.7) (layer F.Cu) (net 1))
 (segment (start 166.85 98.63) (end 160.38 98.63) (width 0.7) (layer F.Cu) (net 1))
 (segment (start 186.03 106.41) (end 186.03 109.91) (width 0.7) (layer F.Cu) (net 1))
 (segment (start 166.85 98.63) (end 178.25 98.63) (width 0.7) (layer F.Cu) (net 1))
 (segment (start 178.25 98.63) (end 186.03 106.41) (width 0.7) (layer F.Cu) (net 1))
 (segment (start 165.98 98.59) (end 169.11 98.59) (width 0.7) (layer B.Cu) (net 1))
 (segment (start 165.04 97.65) (end 165.98 98.59) (width 0.7) (layer B.Cu) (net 1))
 (segment (start 165.04 90.02) (end 165.04 97.65) (width 0.7) (layer B.Cu) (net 1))
 (segment (start 166.63 88.43) (end 165.04 90.02) (width 0.7) (layer B.Cu) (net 1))
 (segment (start 169.11 88.43) (end 166.63 88.43) (width 0.7) (layer B.Cu) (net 1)))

